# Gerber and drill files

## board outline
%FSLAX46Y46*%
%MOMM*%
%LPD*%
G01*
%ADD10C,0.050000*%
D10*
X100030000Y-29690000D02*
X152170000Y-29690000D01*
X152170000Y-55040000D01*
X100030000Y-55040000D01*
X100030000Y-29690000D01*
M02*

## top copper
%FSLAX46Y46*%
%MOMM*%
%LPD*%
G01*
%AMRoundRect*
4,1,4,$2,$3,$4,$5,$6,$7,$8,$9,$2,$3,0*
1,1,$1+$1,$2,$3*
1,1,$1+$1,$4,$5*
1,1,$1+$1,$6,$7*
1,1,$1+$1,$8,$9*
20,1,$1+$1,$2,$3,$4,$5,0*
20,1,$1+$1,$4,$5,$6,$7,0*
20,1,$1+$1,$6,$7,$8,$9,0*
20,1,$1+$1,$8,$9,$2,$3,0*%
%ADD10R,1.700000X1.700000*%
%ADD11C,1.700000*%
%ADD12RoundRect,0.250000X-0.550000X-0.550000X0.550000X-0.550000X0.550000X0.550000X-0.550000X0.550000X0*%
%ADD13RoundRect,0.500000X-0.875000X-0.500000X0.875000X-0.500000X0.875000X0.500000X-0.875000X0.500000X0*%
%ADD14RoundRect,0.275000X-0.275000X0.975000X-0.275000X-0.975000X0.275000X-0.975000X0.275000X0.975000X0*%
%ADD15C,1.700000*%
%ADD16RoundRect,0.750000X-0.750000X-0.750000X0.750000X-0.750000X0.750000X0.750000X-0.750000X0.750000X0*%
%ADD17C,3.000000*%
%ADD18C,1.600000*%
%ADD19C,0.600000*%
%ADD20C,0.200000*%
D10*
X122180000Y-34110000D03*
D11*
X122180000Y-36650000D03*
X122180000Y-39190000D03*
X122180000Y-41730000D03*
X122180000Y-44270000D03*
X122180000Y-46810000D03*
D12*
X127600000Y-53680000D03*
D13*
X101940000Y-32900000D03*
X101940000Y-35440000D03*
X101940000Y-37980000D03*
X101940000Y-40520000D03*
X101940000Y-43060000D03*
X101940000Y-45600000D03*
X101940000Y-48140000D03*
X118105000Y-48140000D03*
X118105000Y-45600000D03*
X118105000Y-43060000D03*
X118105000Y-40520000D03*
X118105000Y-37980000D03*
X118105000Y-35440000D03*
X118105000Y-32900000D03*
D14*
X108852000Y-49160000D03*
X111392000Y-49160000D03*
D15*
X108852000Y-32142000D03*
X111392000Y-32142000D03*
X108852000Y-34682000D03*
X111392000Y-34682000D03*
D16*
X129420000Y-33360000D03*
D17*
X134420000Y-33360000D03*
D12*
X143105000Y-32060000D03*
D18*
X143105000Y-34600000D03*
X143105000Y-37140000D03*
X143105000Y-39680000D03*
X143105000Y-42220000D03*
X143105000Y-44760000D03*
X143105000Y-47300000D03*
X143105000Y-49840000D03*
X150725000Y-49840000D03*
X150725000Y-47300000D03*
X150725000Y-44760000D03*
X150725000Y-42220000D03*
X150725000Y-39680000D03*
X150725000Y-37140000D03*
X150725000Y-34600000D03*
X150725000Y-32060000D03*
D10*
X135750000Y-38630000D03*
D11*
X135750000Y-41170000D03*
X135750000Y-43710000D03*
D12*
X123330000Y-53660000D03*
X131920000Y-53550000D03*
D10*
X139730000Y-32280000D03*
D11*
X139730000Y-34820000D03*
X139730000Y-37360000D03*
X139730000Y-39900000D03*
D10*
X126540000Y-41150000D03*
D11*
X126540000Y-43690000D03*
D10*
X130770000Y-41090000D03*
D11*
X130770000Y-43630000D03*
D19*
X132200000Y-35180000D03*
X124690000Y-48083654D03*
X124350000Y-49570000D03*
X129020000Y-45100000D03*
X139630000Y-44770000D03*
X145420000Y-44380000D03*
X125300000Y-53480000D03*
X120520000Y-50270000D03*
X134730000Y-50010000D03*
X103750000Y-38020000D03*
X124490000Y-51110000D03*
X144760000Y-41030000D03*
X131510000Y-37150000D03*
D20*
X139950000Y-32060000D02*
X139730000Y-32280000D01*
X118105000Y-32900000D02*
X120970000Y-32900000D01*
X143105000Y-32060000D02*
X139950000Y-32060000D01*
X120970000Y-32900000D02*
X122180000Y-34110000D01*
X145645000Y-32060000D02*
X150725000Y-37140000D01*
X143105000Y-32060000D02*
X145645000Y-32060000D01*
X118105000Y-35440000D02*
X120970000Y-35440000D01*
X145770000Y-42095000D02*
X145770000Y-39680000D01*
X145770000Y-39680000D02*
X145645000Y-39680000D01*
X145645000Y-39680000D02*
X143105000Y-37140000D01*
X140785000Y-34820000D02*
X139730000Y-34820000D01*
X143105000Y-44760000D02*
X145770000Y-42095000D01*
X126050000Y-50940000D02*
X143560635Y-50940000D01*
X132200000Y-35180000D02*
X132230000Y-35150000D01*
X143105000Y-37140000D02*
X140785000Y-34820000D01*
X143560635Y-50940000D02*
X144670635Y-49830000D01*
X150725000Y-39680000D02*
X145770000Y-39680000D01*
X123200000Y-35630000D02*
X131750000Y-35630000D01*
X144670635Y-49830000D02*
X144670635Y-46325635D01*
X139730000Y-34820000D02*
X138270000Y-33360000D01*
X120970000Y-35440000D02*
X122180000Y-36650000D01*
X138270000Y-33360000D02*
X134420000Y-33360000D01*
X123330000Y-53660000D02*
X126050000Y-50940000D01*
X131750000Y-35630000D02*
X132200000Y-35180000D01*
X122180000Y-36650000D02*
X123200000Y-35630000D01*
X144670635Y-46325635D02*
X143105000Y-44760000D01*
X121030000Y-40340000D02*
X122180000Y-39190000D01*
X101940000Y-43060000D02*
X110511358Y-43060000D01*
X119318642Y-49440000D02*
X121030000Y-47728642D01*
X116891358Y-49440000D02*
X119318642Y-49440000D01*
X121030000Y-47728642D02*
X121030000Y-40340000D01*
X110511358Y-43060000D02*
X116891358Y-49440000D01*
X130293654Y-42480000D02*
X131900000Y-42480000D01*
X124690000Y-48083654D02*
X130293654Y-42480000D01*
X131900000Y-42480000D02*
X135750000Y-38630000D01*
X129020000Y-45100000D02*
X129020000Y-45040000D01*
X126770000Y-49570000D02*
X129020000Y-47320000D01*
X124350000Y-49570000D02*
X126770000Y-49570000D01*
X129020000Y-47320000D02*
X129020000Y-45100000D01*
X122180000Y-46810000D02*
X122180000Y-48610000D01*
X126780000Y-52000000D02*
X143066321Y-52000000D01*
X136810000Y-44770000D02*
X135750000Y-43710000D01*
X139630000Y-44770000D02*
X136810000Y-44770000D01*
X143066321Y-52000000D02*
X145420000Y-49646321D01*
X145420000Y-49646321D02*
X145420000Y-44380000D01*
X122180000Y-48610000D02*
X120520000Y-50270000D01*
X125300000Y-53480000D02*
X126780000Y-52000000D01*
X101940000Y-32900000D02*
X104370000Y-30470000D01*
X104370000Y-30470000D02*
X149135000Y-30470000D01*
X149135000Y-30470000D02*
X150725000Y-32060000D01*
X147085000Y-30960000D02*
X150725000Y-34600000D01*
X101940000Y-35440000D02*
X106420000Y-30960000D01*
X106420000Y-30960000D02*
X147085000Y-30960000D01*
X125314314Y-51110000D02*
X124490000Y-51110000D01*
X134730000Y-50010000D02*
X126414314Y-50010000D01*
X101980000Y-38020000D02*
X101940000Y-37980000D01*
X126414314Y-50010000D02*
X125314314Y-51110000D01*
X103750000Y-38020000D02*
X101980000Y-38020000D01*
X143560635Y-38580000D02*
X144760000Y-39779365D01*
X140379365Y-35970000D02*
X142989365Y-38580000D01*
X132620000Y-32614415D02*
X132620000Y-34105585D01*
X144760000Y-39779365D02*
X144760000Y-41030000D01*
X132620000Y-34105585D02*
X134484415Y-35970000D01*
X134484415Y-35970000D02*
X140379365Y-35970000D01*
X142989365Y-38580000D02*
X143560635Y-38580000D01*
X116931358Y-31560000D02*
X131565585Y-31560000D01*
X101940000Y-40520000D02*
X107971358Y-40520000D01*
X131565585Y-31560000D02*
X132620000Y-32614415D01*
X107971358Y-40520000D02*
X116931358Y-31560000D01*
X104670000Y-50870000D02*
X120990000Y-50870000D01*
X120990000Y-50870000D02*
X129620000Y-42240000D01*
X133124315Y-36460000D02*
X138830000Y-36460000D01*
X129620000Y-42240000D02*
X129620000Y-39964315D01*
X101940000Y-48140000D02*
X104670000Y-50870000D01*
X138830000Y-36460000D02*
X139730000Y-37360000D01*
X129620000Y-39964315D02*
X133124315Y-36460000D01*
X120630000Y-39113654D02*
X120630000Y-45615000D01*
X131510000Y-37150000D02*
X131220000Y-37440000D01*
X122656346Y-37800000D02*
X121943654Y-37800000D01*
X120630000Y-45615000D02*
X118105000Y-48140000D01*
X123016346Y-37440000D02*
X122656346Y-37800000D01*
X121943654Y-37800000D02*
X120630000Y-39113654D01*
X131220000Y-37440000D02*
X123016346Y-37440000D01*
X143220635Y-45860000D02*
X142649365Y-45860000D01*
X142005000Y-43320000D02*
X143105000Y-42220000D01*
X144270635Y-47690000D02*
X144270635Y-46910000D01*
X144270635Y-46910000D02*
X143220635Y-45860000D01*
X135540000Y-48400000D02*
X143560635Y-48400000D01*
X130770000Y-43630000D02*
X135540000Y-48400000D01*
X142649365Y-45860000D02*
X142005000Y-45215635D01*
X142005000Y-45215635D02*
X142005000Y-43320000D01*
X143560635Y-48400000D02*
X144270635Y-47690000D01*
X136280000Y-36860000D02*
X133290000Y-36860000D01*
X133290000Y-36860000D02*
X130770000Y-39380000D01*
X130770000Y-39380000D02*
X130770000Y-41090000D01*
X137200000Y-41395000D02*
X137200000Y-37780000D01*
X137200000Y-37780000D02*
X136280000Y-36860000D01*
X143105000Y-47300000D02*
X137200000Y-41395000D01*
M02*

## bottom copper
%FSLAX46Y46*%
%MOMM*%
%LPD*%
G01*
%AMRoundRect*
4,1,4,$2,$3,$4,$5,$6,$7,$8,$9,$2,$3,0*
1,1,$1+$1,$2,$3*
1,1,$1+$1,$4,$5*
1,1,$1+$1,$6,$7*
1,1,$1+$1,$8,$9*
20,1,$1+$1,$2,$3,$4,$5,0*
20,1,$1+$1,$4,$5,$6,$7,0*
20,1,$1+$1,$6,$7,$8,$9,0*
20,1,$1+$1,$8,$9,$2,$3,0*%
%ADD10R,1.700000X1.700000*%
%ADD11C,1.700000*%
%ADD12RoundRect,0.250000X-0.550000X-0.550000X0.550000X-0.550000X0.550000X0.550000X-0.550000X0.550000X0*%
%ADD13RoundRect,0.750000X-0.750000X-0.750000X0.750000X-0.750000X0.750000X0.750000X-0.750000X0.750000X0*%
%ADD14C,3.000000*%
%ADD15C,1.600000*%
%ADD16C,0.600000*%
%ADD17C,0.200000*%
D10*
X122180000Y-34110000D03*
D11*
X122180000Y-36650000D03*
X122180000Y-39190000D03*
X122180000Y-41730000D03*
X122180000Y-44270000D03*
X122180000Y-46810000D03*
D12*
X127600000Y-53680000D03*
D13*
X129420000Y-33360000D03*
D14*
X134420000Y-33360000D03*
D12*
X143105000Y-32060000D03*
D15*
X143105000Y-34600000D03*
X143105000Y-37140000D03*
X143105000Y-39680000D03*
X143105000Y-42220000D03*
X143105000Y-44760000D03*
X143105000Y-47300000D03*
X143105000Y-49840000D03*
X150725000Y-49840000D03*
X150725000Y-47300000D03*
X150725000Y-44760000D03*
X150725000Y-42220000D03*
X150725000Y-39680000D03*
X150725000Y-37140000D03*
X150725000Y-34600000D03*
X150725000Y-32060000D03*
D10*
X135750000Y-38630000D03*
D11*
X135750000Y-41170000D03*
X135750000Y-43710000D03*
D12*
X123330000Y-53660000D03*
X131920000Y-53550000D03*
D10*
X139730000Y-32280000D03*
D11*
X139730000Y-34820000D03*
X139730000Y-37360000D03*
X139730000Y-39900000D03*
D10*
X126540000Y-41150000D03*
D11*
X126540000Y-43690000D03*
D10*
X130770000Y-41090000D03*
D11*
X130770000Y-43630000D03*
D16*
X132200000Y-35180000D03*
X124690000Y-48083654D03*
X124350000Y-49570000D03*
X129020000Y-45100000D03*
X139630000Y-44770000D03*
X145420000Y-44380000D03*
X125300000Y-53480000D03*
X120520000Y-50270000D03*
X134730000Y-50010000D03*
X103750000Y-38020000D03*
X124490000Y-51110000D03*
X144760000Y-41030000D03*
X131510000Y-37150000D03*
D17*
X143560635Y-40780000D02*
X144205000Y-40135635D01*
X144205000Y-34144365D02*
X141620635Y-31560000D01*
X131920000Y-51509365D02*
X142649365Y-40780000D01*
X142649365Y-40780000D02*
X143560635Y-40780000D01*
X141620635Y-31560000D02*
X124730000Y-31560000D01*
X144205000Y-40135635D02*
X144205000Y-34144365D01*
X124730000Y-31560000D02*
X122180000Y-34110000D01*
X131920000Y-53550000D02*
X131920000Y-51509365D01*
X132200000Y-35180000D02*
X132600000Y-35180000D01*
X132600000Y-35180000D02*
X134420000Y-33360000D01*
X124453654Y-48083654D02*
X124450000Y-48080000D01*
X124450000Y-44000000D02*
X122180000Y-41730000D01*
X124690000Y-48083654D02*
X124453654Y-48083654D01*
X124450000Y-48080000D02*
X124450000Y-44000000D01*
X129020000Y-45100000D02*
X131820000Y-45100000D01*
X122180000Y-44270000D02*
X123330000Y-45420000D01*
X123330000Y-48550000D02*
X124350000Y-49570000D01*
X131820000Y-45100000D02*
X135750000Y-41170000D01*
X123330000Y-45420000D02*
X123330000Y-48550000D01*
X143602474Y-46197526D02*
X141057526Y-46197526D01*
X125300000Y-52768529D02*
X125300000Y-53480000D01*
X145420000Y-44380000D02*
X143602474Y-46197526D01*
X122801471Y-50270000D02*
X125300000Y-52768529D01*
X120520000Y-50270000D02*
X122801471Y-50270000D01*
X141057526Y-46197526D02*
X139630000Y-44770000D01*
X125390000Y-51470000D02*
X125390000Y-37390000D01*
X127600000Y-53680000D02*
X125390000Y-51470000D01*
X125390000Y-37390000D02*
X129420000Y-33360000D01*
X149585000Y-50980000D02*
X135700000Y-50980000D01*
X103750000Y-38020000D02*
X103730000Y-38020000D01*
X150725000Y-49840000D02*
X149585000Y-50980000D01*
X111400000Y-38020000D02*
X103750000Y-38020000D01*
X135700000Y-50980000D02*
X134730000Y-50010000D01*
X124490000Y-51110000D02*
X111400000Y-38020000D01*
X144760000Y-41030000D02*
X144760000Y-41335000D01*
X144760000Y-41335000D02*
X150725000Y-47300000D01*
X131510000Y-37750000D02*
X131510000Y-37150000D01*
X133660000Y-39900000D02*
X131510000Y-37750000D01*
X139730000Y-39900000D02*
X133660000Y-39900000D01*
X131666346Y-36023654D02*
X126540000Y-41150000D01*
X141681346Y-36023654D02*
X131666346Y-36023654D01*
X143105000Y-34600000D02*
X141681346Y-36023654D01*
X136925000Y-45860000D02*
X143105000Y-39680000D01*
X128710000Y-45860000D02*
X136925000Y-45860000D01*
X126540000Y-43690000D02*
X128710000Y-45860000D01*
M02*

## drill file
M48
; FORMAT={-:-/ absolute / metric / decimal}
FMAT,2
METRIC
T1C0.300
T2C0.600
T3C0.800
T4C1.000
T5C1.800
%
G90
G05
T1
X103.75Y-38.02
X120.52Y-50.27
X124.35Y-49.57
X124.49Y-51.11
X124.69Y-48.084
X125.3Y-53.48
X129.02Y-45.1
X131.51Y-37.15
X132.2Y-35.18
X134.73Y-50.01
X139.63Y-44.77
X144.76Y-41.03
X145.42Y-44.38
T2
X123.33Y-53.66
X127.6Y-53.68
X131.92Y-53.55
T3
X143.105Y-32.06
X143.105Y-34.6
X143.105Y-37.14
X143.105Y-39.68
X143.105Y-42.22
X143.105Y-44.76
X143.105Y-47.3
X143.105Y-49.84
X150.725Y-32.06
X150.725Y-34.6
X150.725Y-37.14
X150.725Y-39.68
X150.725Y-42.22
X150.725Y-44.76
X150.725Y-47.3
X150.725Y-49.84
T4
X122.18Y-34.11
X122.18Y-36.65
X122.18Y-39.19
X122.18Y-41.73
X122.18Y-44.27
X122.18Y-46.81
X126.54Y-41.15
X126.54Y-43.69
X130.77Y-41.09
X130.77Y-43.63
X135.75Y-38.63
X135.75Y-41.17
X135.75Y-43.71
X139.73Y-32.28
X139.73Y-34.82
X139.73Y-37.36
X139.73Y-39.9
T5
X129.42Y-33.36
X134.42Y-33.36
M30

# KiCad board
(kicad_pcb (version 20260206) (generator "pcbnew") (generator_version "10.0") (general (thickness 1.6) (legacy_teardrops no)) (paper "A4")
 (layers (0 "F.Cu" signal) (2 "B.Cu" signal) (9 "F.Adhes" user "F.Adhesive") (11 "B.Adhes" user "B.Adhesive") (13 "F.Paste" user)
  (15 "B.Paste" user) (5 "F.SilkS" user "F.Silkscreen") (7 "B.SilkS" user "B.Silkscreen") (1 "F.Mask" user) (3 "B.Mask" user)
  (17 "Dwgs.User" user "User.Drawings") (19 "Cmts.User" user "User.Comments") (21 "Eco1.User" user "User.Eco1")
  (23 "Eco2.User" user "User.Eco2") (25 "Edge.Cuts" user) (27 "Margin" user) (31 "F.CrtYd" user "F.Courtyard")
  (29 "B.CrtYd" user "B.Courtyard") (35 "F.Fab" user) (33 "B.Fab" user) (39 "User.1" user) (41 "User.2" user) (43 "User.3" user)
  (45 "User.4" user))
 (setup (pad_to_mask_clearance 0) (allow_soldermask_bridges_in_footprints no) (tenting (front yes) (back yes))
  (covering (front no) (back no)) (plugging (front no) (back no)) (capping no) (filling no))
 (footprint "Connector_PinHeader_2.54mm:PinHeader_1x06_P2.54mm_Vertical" (layer "F.Cu") (at 122.18 34.11)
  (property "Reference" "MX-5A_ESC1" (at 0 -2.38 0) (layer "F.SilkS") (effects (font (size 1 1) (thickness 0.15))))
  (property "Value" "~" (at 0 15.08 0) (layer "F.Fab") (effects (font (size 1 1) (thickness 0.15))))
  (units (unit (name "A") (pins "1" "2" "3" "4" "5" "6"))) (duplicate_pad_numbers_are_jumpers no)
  (pad "1" thru_hole rect (at 0 0) (size 1.7 1.7) (drill 1) (layers "*.Cu" "*.Mask") (remove_unused_layers no) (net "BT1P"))
  (pad "2" thru_hole circle (at 0 2.54) (size 1.7 1.7) (drill 1) (layers "*.Cu" "*.Mask") (remove_unused_layers no) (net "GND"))
  (pad "3" thru_hole circle (at 0 5.08) (size 1.7 1.7) (drill 1) (layers "*.Cu" "*.Mask") (remove_unused_layers no)
   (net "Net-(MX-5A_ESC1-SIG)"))
  (pad "4" thru_hole circle (at 0 7.62) (size 1.7 1.7) (drill 1) (layers "*.Cu" "*.Mask") (remove_unused_layers no)
   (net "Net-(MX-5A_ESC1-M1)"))
  (pad "5" thru_hole circle (at 0 10.16) (size 1.7 1.7) (drill 1) (layers "*.Cu" "*.Mask") (remove_unused_layers no)
   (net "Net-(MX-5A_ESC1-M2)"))
  (pad "6" thru_hole circle (at 0 12.7) (size 1.7 1.7) (drill 1) (layers "*.Cu" "*.Mask") (remove_unused_layers no)
   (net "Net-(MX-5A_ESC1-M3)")))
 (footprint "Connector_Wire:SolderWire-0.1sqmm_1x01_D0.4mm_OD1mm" (layer "F.Cu") (at 127.6 53.68)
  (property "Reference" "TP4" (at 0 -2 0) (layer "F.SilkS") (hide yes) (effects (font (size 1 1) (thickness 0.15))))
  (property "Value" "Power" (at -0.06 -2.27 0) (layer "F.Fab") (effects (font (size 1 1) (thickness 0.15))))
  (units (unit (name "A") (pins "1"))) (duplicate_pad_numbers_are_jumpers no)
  (pad "1" thru_hole roundrect (at 0 0) (size 1.6 1.6) (drill 0.6) (layers "*.Cu" "*.Mask") (remove_unused_layers no)
   (roundrect_rratio 0.15625) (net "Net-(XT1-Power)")))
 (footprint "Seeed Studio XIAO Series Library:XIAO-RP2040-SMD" (layer "F.Cu") (at 109.94 40.52)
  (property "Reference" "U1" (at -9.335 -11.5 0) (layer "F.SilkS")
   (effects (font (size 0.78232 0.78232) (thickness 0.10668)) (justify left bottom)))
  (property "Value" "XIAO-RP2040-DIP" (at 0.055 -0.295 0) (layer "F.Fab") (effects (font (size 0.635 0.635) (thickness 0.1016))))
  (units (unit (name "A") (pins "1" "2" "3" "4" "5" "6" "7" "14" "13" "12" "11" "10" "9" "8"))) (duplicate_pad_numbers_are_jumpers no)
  (pad "1" smd roundrect (at -8 -7.62) (size 2.75 2) (layers "F.Cu" "F.Mask" "F.Paste") (roundrect_rratio 0.25) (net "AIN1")
   (solder_mask_margin 0.0508) (thermal_bridge_angle 45))
  (pad "2" smd roundrect (at -8 -5.08) (size 2.75 2) (layers "F.Cu" "F.Mask" "F.Paste") (roundrect_rratio 0.25) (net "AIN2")
   (solder_mask_margin 0.0508) (thermal_bridge_angle 45))
  (pad "3" smd roundrect (at -8 -2.54) (size 2.75 2) (layers "F.Cu" "F.Mask" "F.Paste") (roundrect_rratio 0.25) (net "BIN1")
   (solder_mask_margin 0.0508) (thermal_bridge_angle 45))
  (pad "4" smd roundrect (at -8 0) (size 2.75 2) (layers "F.Cu" "F.Mask" "F.Paste") (roundrect_rratio 0.25) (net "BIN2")
   (solder_mask_margin 0.0508) (thermal_bridge_angle 45))
  (pad "5" smd roundrect (at -8 2.54) (size 2.75 2) (layers "F.Cu" "F.Mask" "F.Paste") (roundrect_rratio 0.25) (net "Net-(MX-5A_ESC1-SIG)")
   (solder_mask_margin 0.0508) (thermal_bridge_angle 45))
  (pad "6" smd roundrect (at -8 5.08) (size 2.75 2) (layers "F.Cu" "F.Mask" "F.Paste") (roundrect_rratio 0.25)
   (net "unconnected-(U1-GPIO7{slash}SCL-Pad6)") (solder_mask_margin 0.0508) (thermal_bridge_angle 45))
  (pad "7" smd roundrect (at -8 7.62) (size 2.75 2) (layers "F.Cu" "F.Mask" "F.Paste") (roundrect_rratio 0.25)
   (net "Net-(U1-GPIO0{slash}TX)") (solder_mask_margin 0.0508) (thermal_bridge_angle 45))
  (pad "8" smd roundrect (at 8.165 7.62) (size 2.75 2) (layers "F.Cu" "F.Mask" "F.Paste") (roundrect_rratio 0.25)
   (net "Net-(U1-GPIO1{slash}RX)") (solder_mask_margin 0.0508) (thermal_bridge_angle 45))
  (pad "9" smd roundrect (at 8.165 5.08) (size 2.75 2) (layers "F.Cu" "F.Mask" "F.Paste") (roundrect_rratio 0.25)
   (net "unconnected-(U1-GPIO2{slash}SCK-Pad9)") (solder_mask_margin 0.0508) (thermal_bridge_angle 45))
  (pad "10" smd roundrect (at 8.165 2.54) (size 2.75 2) (layers "F.Cu" "F.Mask" "F.Paste") (roundrect_rratio 0.25)
   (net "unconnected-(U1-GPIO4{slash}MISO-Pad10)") (solder_mask_margin 0.0508) (thermal_bridge_angle 45))
  (pad "11" smd roundrect (at 8.165 0) (size 2.75 2) (layers "F.Cu" "F.Mask" "F.Paste") (roundrect_rratio 0.25)
   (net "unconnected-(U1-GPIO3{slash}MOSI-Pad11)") (solder_mask_margin 0.0508) (thermal_bridge_angle 45))
  (pad "12" smd roundrect (at 8.165 -2.54) (size 2.75 2) (layers "F.Cu" "F.Mask" "F.Paste") (roundrect_rratio 0.25)
   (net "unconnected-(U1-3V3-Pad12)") (solder_mask_margin 0.0508) (thermal_bridge_angle 45))
  (pad "13" smd roundrect (at 8.165 -5.08) (size 2.75 2) (layers "F.Cu" "F.Mask" "F.Paste") (roundrect_rratio 0.25) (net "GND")
   (solder_mask_margin 0.0508) (thermal_bridge_angle 45))
  (pad "14" smd roundrect (at 8.165 -7.62) (size 2.75 2) (layers "F.Cu" "F.Mask" "F.Paste") (roundrect_rratio 0.25) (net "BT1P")
   (solder_mask_margin 0.0508) (thermal_bridge_angle 45))
  (pad "15" smd roundrect (at -1.088 8.64 270) (size 2.5 1.1) (layers "F.Cu" "F.Mask" "F.Paste") (roundrect_rratio 0.25)
   (thermal_bridge_angle 45))
  (pad "16" smd roundrect (at 1.452 8.64 270) (size 2.5 1.1) (layers "F.Cu" "F.Mask" "F.Paste") (roundrect_rratio 0.25)
   (thermal_bridge_angle 45))
  (pad "17" smd circle (at -1.088 -8.378) (size 1.7 1.7) (layers "F.Cu" "F.Mask" "F.Paste"))
  (pad "18" smd circle (at 1.452 -8.378) (size 1.7 1.7) (layers "F.Cu" "F.Mask" "F.Paste"))
  (pad "19" smd circle (at -1.088 -5.838) (size 1.7 1.7) (layers "F.Cu" "F.Mask" "F.Paste"))
  (pad "20" smd circle (at 1.452 -5.838) (size 1.7 1.7) (layers "F.Cu" "F.Mask" "F.Paste")))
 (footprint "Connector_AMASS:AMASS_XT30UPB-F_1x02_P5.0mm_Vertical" (layer "F.Cu") (at 129.42 33.36)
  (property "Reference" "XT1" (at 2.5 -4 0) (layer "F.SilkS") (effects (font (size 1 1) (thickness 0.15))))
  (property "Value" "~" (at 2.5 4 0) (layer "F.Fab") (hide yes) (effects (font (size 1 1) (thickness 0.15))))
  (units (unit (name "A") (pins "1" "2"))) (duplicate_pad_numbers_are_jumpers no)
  (pad "1" thru_hole roundrect (at 0 0) (size 3 3) (drill 1.8) (layers "*.Cu" "*.Mask") (remove_unused_layers no) (roundrect_rratio 0.25)
   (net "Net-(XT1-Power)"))
  (pad "2" thru_hole circle (at 5 0) (size 3 3) (drill 1.8) (layers "*.Cu" "*.Mask") (remove_unused_layers no) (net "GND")))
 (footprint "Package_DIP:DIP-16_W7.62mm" (layer "F.Cu") (at 143.105 32.06)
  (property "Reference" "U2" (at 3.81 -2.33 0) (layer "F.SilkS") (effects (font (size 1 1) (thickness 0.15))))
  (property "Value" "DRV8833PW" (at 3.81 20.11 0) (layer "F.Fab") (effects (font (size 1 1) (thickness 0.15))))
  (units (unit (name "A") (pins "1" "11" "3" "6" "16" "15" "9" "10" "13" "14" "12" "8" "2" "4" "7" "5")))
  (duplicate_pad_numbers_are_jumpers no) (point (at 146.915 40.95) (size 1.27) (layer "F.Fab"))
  (pad "1" thru_hole roundrect (at 0 0) (size 1.6 1.6) (drill 0.8) (layers "*.Cu" "*.Mask") (remove_unused_layers no)
   (roundrect_rratio 0.15625) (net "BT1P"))
  (pad "2" thru_hole circle (at 0 2.54) (size 1.6 1.6) (drill 0.8) (layers "*.Cu" "*.Mask") (remove_unused_layers no) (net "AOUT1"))
  (pad "3" thru_hole circle (at 0 5.08) (size 1.6 1.6) (drill 0.8) (layers "*.Cu" "*.Mask") (remove_unused_layers no) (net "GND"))
  (pad "4" thru_hole circle (at 0 7.62) (size 1.6 1.6) (drill 0.8) (layers "*.Cu" "*.Mask") (remove_unused_layers no) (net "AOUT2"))
  (pad "5" thru_hole circle (at 0 10.16) (size 1.6 1.6) (drill 0.8) (layers "*.Cu" "*.Mask") (remove_unused_layers no) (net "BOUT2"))
  (pad "6" thru_hole circle (at 0 12.7) (size 1.6 1.6) (drill 0.8) (layers "*.Cu" "*.Mask") (remove_unused_layers no) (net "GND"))
  (pad "7" thru_hole circle (at 0 15.24) (size 1.6 1.6) (drill 0.8) (layers "*.Cu" "*.Mask") (remove_unused_layers no) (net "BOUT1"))
  (pad "8" thru_hole circle (at 0 17.78) (size 1.6 1.6) (drill 0.8) (layers "*.Cu" "*.Mask") (remove_unused_layers no)
   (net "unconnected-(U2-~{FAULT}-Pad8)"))
  (pad "9" thru_hole circle (at 7.62 17.78) (size 1.6 1.6) (drill 0.8) (layers "*.Cu" "*.Mask") (remove_unused_layers no) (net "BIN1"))
  (pad "10" thru_hole circle (at 7.62 15.24) (size 1.6 1.6) (drill 0.8) (layers "*.Cu" "*.Mask") (remove_unused_layers no) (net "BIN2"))
  (pad "11" thru_hole circle (at 7.62 12.7) (size 1.6 1.6) (drill 0.8) (layers "*.Cu" "*.Mask") (remove_unused_layers no)
   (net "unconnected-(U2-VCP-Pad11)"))
  (pad "12" thru_hole circle (at 7.62 10.16) (size 1.6 1.6) (drill 0.8) (layers "*.Cu" "*.Mask") (remove_unused_layers no)
   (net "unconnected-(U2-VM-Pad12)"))
  (pad "13" thru_hole circle (at 7.62 7.62) (size 1.6 1.6) (drill 0.8) (layers "*.Cu" "*.Mask") (remove_unused_layers no) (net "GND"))
  (pad "14" thru_hole circle (at 7.62 5.08) (size 1.6 1.6) (drill 0.8) (layers "*.Cu" "*.Mask") (remove_unused_layers no) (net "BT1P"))
  (pad "15" thru_hole circle (at 7.62 2.54) (size 1.6 1.6) (drill 0.8) (layers "*.Cu" "*.Mask") (remove_unused_layers no) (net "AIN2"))
  (pad "16" thru_hole circle (at 7.62 0) (size 1.6 1.6) (drill 0.8) (layers "*.Cu" "*.Mask") (remove_unused_layers no) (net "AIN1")))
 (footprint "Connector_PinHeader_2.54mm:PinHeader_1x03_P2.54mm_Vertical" (layer "F.Cu") (at 135.75 38.63)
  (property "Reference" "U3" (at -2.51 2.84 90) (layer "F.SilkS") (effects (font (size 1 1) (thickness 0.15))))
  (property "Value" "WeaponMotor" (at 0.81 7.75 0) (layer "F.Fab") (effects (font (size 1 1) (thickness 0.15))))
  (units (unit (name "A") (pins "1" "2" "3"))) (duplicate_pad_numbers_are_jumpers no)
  (pad "1" thru_hole rect (at 0 0) (size 1.7 1.7) (drill 1) (layers "*.Cu" "*.Mask") (remove_unused_layers no) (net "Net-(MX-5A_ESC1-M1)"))
  (pad "2" thru_hole circle (at 0 2.54) (size 1.7 1.7) (drill 1) (layers "*.Cu" "*.Mask") (remove_unused_layers no)
   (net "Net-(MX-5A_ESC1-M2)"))
  (pad "3" thru_hole circle (at 0 5.08) (size 1.7 1.7) (drill 1) (layers "*.Cu" "*.Mask") (remove_unused_layers no)
   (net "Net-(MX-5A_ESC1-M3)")))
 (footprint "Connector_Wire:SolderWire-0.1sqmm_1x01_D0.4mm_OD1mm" (layer "F.Cu") (at 123.33 53.66)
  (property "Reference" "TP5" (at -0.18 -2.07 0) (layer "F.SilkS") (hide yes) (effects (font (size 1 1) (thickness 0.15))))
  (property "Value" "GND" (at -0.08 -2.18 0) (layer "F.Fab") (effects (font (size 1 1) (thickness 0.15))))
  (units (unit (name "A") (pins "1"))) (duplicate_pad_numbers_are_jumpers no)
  (pad "1" thru_hole roundrect (at 0 0) (size 1.6 1.6) (drill 0.6) (layers "*.Cu" "*.Mask") (remove_unused_layers no)
   (roundrect_rratio 0.15625) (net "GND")))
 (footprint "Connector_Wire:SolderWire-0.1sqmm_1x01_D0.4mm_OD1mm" (layer "F.Cu") (at 131.92 53.55)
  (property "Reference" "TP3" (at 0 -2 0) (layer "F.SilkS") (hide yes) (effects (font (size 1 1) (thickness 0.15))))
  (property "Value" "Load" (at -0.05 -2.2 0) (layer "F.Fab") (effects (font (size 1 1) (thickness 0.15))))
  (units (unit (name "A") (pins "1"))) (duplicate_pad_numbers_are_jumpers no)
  (pad "1" thru_hole roundrect (at 0 0) (size 1.6 1.6) (drill 0.6) (layers "*.Cu" "*.Mask") (remove_unused_layers no)
   (roundrect_rratio 0.15625) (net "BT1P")))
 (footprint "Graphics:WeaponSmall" (layer "F.Cu") (at 103.49791 55.032445 90)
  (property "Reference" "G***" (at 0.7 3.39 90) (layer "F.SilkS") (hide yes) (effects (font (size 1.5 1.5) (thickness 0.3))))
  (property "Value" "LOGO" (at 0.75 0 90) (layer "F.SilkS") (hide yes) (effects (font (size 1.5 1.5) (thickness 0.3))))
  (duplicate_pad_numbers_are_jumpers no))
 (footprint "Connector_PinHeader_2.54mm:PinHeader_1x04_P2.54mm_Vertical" (layer "F.Cu") (at 139.73 32.28)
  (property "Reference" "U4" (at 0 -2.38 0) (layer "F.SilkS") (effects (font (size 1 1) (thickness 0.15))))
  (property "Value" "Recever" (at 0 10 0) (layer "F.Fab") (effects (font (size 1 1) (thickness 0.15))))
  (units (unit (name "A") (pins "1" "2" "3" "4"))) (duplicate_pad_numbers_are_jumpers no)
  (pad "1" thru_hole rect (at 0 0) (size 1.7 1.7) (drill 1) (layers "*.Cu" "*.Mask") (remove_unused_layers no) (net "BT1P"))
  (pad "2" thru_hole circle (at 0 2.54) (size 1.7 1.7) (drill 1) (layers "*.Cu" "*.Mask") (remove_unused_layers no) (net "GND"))
  (pad "3" thru_hole circle (at 0 5.08) (size 1.7 1.7) (drill 1) (layers "*.Cu" "*.Mask") (remove_unused_layers no)
   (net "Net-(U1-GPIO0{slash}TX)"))
  (pad "4" thru_hole circle (at 0 7.62) (size 1.7 1.7) (drill 1) (layers "*.Cu" "*.Mask") (remove_unused_layers no)
   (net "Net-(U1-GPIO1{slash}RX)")))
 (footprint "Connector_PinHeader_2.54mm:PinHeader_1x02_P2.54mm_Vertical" (layer "F.Cu") (at 126.54 41.15)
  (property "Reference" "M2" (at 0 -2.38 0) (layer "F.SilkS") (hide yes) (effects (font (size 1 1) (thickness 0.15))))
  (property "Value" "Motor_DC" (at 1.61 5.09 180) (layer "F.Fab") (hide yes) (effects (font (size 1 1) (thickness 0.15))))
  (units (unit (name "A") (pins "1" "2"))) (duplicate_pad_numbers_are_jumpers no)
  (pad "1" thru_hole rect (at 0 0) (size 1.7 1.7) (drill 1) (layers "*.Cu" "*.Mask") (remove_unused_layers no) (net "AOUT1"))
  (pad "2" thru_hole circle (at 0 2.54) (size 1.7 1.7) (drill 1) (layers "*.Cu" "*.Mask") (remove_unused_layers no) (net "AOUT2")))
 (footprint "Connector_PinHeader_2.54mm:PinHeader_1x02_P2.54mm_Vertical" (layer "F.Cu") (at 130.77 41.09)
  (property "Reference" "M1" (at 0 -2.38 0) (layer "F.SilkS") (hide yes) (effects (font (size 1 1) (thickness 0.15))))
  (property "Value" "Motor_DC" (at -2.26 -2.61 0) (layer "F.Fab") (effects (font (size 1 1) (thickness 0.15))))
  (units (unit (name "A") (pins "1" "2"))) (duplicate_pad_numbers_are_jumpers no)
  (pad "1" thru_hole rect (at 0 0) (size 1.7 1.7) (drill 1) (layers "*.Cu" "*.Mask") (remove_unused_layers no) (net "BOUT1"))
  (pad "2" thru_hole circle (at 0 2.54) (size 1.7 1.7) (drill 1) (layers "*.Cu" "*.Mask") (remove_unused_layers no) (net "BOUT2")))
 (gr_rect (start 100.03 29.69) (end 152.17 55.04) (stroke (width 0.05) (type default)) (fill no) (layer "Edge.Cuts"))
 (segment (start 139.95 32.06) (end 139.73 32.28) (width 0.2) (layer "F.Cu") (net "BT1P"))
 (segment (start 118.105 32.9) (end 120.97 32.9) (width 0.2) (layer "F.Cu") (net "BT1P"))
 (segment (start 143.105 32.06) (end 139.95 32.06) (width 0.2) (layer "F.Cu") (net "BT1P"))
 (segment (start 120.97 32.9) (end 122.18 34.11) (width 0.2) (layer "F.Cu") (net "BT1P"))
 (segment (start 145.645 32.06) (end 150.725 37.14) (width 0.2) (layer "F.Cu") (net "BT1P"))
 (segment (start 143.105 32.06) (end 145.645 32.06) (width 0.2) (layer "F.Cu") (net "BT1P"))
 (segment (start 143.560635 40.78) (end 144.205 40.135635) (width 0.2) (layer "B.Cu") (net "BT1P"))
 (segment (start 144.205 34.144365) (end 141.620635 31.56) (width 0.2) (layer "B.Cu") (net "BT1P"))
 (segment (start 131.92 51.509365) (end 142.649365 40.78) (width 0.2) (layer "B.Cu") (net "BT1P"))
 (segment (start 142.649365 40.78) (end 143.560635 40.78) (width 0.2) (layer "B.Cu") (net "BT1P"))
 (segment (start 141.620635 31.56) (end 124.73 31.56) (width 0.2) (layer "B.Cu") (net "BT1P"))
 (segment (start 144.205 40.135635) (end 144.205 34.144365) (width 0.2) (layer "B.Cu") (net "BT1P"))
 (segment (start 124.73 31.56) (end 122.18 34.11) (width 0.2) (layer "B.Cu") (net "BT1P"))
 (segment (start 131.92 53.55) (end 131.92 51.509365) (width 0.2) (layer "B.Cu") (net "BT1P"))
 (segment (start 118.105 35.44) (end 120.97 35.44) (width 0.2) (layer "F.Cu") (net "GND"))
 (segment (start 145.77 42.095) (end 145.77 39.68) (width 0.2) (layer "F.Cu") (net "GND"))
 (segment (start 145.77 39.68) (end 145.645 39.68) (width 0.2) (layer "F.Cu") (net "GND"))
 (segment (start 145.645 39.68) (end 143.105 37.14) (width 0.2) (layer "F.Cu") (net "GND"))
 (segment (start 140.785 34.82) (end 139.73 34.82) (width 0.2) (layer "F.Cu") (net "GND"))
 (segment (start 143.105 44.76) (end 145.77 42.095) (width 0.2) (layer "F.Cu") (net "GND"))
 (segment (start 126.05 50.94) (end 143.560635 50.94) (width 0.2) (layer "F.Cu") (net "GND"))
 (segment (start 132.2 35.18) (end 132.23 35.15) (width 0.2) (layer "F.Cu") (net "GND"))
 (segment (start 143.105 37.14) (end 140.785 34.82) (width 0.2) (layer "F.Cu") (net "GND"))
 (segment (start 143.560635 50.94) (end 144.670635 49.83) (width 0.2) (layer "F.Cu") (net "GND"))
 (segment (start 150.725 39.68) (end 145.77 39.68) (width 0.2) (layer "F.Cu") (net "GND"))
 (segment (start 123.2 35.63) (end 131.75 35.63) (width 0.2) (layer "F.Cu") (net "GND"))
 (segment (start 144.670635 49.83) (end 144.670635 46.325635) (width 0.2) (layer "F.Cu") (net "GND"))
 (segment (start 139.73 34.82) (end 138.27 33.36) (width 0.2) (layer "F.Cu") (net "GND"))
 (segment (start 120.97 35.44) (end 122.18 36.65) (width 0.2) (layer "F.Cu") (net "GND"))
 (segment (start 138.27 33.36) (end 134.42 33.36) (width 0.2) (layer "F.Cu") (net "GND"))
 (segment (start 123.33 53.66) (end 126.05 50.94) (width 0.2) (layer "F.Cu") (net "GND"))
 (segment (start 131.75 35.63) (end 132.2 35.18) (width 0.2) (layer "F.Cu") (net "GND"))
 (segment (start 122.18 36.65) (end 123.2 35.63) (width 0.2) (layer "F.Cu") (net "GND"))
 (segment (start 144.670635 46.325635) (end 143.105 44.76) (width 0.2) (layer "F.Cu") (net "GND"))
 (via (at 132.2 35.18) (size 0.6) (drill 0.3) (layers "F.Cu" "B.Cu") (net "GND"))
 (segment (start 132.2 35.18) (end 132.6 35.18) (width 0.2) (layer "B.Cu") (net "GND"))
 (segment (start 132.6 35.18) (end 134.42 33.36) (width 0.2) (layer "B.Cu") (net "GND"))
 (segment (start 121.03 40.34) (end 122.18 39.19) (width 0.2) (layer "F.Cu") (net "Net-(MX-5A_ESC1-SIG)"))
 (segment (start 101.94 43.06) (end 110.511358 43.06) (width 0.2) (layer "F.Cu") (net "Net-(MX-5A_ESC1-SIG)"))
 (segment (start 119.318642 49.44) (end 121.03 47.728642) (width 0.2) (layer "F.Cu") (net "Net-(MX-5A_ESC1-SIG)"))
 (segment (start 116.891358 49.44) (end 119.318642 49.44) (width 0.2) (layer "F.Cu") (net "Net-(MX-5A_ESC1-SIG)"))
 (segment (start 121.03 47.728642) (end 121.03 40.34) (width 0.2) (layer "F.Cu") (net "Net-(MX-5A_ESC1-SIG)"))
 (segment (start 110.511358 43.06) (end 116.891358 49.44) (width 0.2) (layer "F.Cu") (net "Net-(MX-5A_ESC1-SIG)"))
 (segment (start 130.293654 42.48) (end 131.9 42.48) (width 0.2) (layer "F.Cu") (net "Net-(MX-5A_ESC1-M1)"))
 (segment (start 124.69 48.083654) (end 130.293654 42.48) (width 0.2) (layer "F.Cu") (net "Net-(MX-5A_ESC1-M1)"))
 (segment (start 131.9 42.48) (end 135.75 38.63) (width 0.2) (layer "F.Cu") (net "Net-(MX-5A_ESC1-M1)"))
 (via (at 124.69 48.083654) (size 0.6) (drill 0.3) (layers "F.Cu" "B.Cu") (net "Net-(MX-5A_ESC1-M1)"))
 (segment (start 124.453654 48.083654) (end 124.45 48.08) (width 0.2) (layer "B.Cu") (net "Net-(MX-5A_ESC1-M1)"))
 (segment (start 124.45 44) (end 122.18 41.73) (width 0.2) (layer "B.Cu") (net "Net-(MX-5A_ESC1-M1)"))
 (segment (start 124.69 48.083654) (end 124.453654 48.083654) (width 0.2) (layer "B.Cu") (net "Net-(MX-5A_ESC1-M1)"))
 (segment (start 124.45 48.08) (end 124.45 44) (width 0.2) (layer "B.Cu") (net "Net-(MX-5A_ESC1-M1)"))
 (segment (start 129.02 45.1) (end 129.02 45.04) (width 0.2) (layer "F.Cu") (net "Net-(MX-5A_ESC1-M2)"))
 (segment (start 126.77 49.57) (end 129.02 47.32) (width 0.2) (layer "F.Cu") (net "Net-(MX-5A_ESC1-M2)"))
 (segment (start 124.35 49.57) (end 126.77 49.57) (width 0.2) (layer "F.Cu") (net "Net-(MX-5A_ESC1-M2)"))
 (segment (start 129.02 47.32) (end 129.02 45.1) (width 0.2) (layer "F.Cu") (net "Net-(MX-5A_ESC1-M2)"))
 (via (at 124.35 49.57) (size 0.6) (drill 0.3) (layers "F.Cu" "B.Cu") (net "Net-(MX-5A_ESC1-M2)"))
 (via (at 129.02 45.1) (size 0.6) (drill 0.3) (layers "F.Cu" "B.Cu") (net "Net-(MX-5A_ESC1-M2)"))
 (segment (start 129.02 45.1) (end 131.82 45.1) (width 0.2) (layer "B.Cu") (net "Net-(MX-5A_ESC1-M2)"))
 (segment (start 122.18 44.27) (end 123.33 45.42) (width 0.2) (layer "B.Cu") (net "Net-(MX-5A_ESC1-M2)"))
 (segment (start 123.33 48.55) (end 124.35 49.57) (width 0.2) (layer "B.Cu") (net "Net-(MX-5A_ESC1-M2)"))
 (segment (start 131.82 45.1) (end 135.75 41.17) (width 0.2) (layer "B.Cu") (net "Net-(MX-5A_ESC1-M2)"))
 (segment (start 123.33 45.42) (end 123.33 48.55) (width 0.2) (layer "B.Cu") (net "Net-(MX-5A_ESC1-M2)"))
 (segment (start 122.18 46.81) (end 122.18 48.61) (width 0.2) (layer "F.Cu") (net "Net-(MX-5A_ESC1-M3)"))
 (segment (start 126.78 52) (end 143.066321 52) (width 0.2) (layer "F.Cu") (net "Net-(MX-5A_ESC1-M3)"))
 (segment (start 136.81 44.77) (end 135.75 43.71) (width 0.2) (layer "F.Cu") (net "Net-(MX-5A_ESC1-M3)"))
 (segment (start 139.63 44.77) (end 136.81 44.77) (width 0.2) (layer "F.Cu") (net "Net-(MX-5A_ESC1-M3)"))
 (segment (start 143.066321 52) (end 145.42 49.646321) (width 0.2) (layer "F.Cu") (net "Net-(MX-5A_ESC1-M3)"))
 (segment (start 145.42 49.646321) (end 145.42 44.38) (width 0.2) (layer "F.Cu") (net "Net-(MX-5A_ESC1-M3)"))
 (segment (start 122.18 48.61) (end 120.52 50.27) (width 0.2) (layer "F.Cu") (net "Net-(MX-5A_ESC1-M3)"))
 (segment (start 125.3 53.48) (end 126.78 52) (width 0.2) (layer "F.Cu") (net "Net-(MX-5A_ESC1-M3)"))
 (via (at 139.63 44.77) (size 0.6) (drill 0.3) (layers "F.Cu" "B.Cu") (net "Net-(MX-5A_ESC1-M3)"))
 (via (at 145.42 44.38) (size 0.6) (drill 0.3) (layers "F.Cu" "B.Cu") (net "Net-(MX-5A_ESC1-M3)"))
 (via (at 125.3 53.48) (size 0.6) (drill 0.3) (layers "F.Cu" "B.Cu") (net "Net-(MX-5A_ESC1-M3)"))
 (via (at 120.52 50.27) (size 0.6) (drill 0.3) (layers "F.Cu" "B.Cu") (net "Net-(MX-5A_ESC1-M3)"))
 (segment (start 143.602474 46.197526) (end 141.057526 46.197526) (width 0.2) (layer "B.Cu") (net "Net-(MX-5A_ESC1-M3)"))
 (segment (start 125.3 52.768529) (end 125.3 53.48) (width 0.2) (layer "B.Cu") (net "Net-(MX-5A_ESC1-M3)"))
 (segment (start 145.42 44.38) (end 143.602474 46.197526) (width 0.2) (layer "B.Cu") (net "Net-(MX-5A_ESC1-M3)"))
 (segment (start 122.801471 50.27) (end 125.3 52.768529) (width 0.2) (layer "B.Cu") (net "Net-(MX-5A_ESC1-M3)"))
 (segment (start 120.52 50.27) (end 122.801471 50.27) (width 0.2) (layer "B.Cu") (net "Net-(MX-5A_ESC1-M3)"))
 (segment (start 141.057526 46.197526) (end 139.63 44.77) (width 0.2) (layer "B.Cu") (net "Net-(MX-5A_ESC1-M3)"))
 (segment (start 125.39 51.47) (end 125.39 37.39) (width 0.2) (layer "B.Cu") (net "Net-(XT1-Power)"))
 (segment (start 127.6 53.68) (end 125.39 51.47) (width 0.2) (layer "B.Cu") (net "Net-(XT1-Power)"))
 (segment (start 125.39 37.39) (end 129.42 33.36) (width 0.2) (layer "B.Cu") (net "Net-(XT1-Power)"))
 (segment (start 101.94 32.9) (end 104.37 30.47) (width 0.2) (layer "F.Cu") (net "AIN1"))
 (segment (start 104.37 30.47) (end 149.135 30.47) (width 0.2) (layer "F.Cu") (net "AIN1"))
 (segment (start 149.135 30.47) (end 150.725 32.06) (width 0.2) (layer "F.Cu") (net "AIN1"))
 (segment (start 147.085 30.96) (end 150.725 34.6) (width 0.2) (layer "F.Cu") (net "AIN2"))
 (segment (start 101.94 35.44) (end 106.42 30.96) (width 0.2) (layer "F.Cu") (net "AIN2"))
 (segment (start 106.42 30.96) (end 147.085 30.96) (width 0.2) (layer "F.Cu") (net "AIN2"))
 (segment (start 125.314314 51.11) (end 124.49 51.11) (width 0.2) (layer "F.Cu") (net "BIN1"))
 (segment (start 134.73 50.01) (end 126.414314 50.01) (width 0.2) (layer "F.Cu") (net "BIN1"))
 (segment (start 101.98 38.02) (end 101.94 37.98) (width 0.2) (layer "F.Cu") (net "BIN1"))
 (segment (start 126.414314 50.01) (end 125.314314 51.11) (width 0.2) (layer "F.Cu") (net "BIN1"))
 (segment (start 103.75 38.02) (end 101.98 38.02) (width 0.2) (layer "F.Cu") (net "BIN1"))
 (via (at 134.73 50.01) (size 0.6) (drill 0.3) (layers "F.Cu" "B.Cu") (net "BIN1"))
 (via (at 103.75 38.02) (size 0.6) (drill 0.3) (layers "F.Cu" "B.Cu") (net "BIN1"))
 (via (at 124.49 51.11) (size 0.6) (drill 0.3) (layers "F.Cu" "B.Cu") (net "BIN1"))
 (segment (start 149.585 50.98) (end 135.7 50.98) (width 0.2) (layer "B.Cu") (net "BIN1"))
 (segment (start 103.75 38.02) (end 103.73 38.02) (width 0.2) (layer "B.Cu") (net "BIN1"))
 (segment (start 150.725 49.84) (end 149.585 50.98) (width 0.2) (layer "B.Cu") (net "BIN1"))
 (segment (start 111.4 38.02) (end 103.75 38.02) (width 0.2) (layer "B.Cu") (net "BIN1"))
 (segment (start 135.7 50.98) (end 134.73 50.01) (width 0.2) (layer "B.Cu") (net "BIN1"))
 (segment (start 124.49 51.11) (end 111.4 38.02) (width 0.2) (layer "B.Cu") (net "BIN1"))
 (segment (start 143.560635 38.58) (end 144.76 39.779365) (width 0.2) (layer "F.Cu") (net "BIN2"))
 (segment (start 140.379365 35.97) (end 142.989365 38.58) (width 0.2) (layer "F.Cu") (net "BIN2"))
 (segment (start 132.62 32.614415) (end 132.62 34.105585) (width 0.2) (layer "F.Cu") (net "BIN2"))
 (segment (start 144.76 39.779365) (end 144.76 41.03) (width 0.2) (layer "F.Cu") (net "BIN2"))
 (segment (start 132.62 34.105585) (end 134.484415 35.97) (width 0.2) (layer "F.Cu") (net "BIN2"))
 (segment (start 134.484415 35.97) (end 140.379365 35.97) (width 0.2) (layer "F.Cu") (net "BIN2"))
 (segment (start 142.989365 38.58) (end 143.560635 38.58) (width 0.2) (layer "F.Cu") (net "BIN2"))
 (segment (start 116.931358 31.56) (end 131.565585 31.56) (width 0.2) (layer "F.Cu") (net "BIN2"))
 (segment (start 101.94 40.52) (end 107.971358 40.52) (width 0.2) (layer "F.Cu") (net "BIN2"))
 (segment (start 131.565585 31.56) (end 132.62 32.614415) (width 0.2) (layer "F.Cu") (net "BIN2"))
 (segment (start 107.971358 40.52) (end 116.931358 31.56) (width 0.2) (layer "F.Cu") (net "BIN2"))
 (via (at 144.76 41.03) (size 0.6) (drill 0.3) (layers "F.Cu" "B.Cu") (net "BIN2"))
 (segment (start 144.76 41.03) (end 144.76 41.335) (width 0.2) (layer "B.Cu") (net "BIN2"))
 (segment (start 144.76 41.335) (end 150.725 47.3) (width 0.2) (layer "B.Cu") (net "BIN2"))
 (segment (start 104.67 50.87) (end 120.99 50.87) (width 0.2) (layer "F.Cu") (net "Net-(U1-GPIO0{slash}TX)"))
 (segment (start 120.99 50.87) (end 129.62 42.24) (width 0.2) (layer "F.Cu") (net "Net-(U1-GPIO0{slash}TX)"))
 (segment (start 133.124315 36.46) (end 138.83 36.46) (width 0.2) (layer "F.Cu") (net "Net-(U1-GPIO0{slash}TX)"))
 (segment (start 129.62 42.24) (end 129.62 39.964315) (width 0.2) (layer "F.Cu") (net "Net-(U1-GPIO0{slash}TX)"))
 (segment (start 101.94 48.14) (end 104.67 50.87) (width 0.2) (layer "F.Cu") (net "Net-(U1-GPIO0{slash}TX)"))
 (segment (start 138.83 36.46) (end 139.73 37.36) (width 0.2) (layer "F.Cu") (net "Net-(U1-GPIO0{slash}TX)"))
 (segment (start 129.62 39.964315) (end 133.124315 36.46) (width 0.2) (layer "F.Cu") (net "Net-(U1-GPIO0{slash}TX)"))
 (segment (start 120.63 39.113654) (end 120.63 45.615) (width 0.2) (layer "F.Cu") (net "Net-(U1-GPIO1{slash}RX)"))
 (segment (start 131.51 37.15) (end 131.22 37.44) (width 0.2) (layer "F.Cu") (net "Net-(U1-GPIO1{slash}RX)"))
 (segment (start 122.656346 37.8) (end 121.943654 37.8) (width 0.2) (layer "F.Cu") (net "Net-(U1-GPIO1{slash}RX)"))
 (segment (start 120.63 45.615) (end 118.105 48.14) (width 0.2) (layer "F.Cu") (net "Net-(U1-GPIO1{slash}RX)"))
 (segment (start 123.016346 37.44) (end 122.656346 37.8) (width 0.2) (layer "F.Cu") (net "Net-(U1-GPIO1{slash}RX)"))
 (segment (start 121.943654 37.8) (end 120.63 39.113654) (width 0.2) (layer "F.Cu") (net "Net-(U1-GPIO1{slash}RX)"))
 (segment (start 131.22 37.44) (end 123.016346 37.44) (width 0.2) (layer "F.Cu") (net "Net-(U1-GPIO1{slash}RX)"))
 (via (at 131.51 37.15) (size 0.6) (drill 0.3) (layers "F.Cu" "B.Cu") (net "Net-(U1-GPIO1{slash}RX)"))
 (segment (start 131.51 37.75) (end 131.51 37.15) (width 0.2) (layer "B.Cu") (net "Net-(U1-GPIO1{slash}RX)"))
 (segment (start 133.66 39.9) (end 131.51 37.75) (width 0.2) (layer "B.Cu") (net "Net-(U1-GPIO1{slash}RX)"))
 (segment (start 139.73 39.9) (end 133.66 39.9) (width 0.2) (layer "B.Cu") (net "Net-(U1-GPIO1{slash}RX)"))
 (segment (start 131.666346 36.023654) (end 126.54 41.15) (width 0.2) (layer "B.Cu") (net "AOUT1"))
 (segment (start 141.681346 36.023654) (end 131.666346 36.023654) (width 0.2) (layer "B.Cu") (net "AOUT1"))
 (segment (start 143.105 34.6) (end 141.681346 36.023654) (width 0.2) (layer "B.Cu") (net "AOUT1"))
 (segment (start 136.925 45.86) (end 143.105 39.68) (width 0.2) (layer "B.Cu") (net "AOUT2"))
 (segment (start 128.71 45.86) (end 136.925 45.86) (width 0.2) (layer "B.Cu") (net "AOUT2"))
 (segment (start 126.54 43.69) (end 128.71 45.86) (width 0.2) (layer "B.Cu") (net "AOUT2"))
 (segment (start 143.220635 45.86) (end 142.649365 45.86) (width 0.2) (layer "F.Cu") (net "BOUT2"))
 (segment (start 142.005 43.32) (end 143.105 42.22) (width 0.2) (layer "F.Cu") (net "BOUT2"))
 (segment (start 144.270635 47.69) (end 144.270635 46.91) (width 0.2) (layer "F.Cu") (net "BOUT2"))
 (segment (start 144.270635 46.91) (end 143.220635 45.86) (width 0.2) (layer "F.Cu") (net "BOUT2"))
 (segment (start 135.54 48.4) (end 143.560635 48.4) (width 0.2) (layer "F.Cu") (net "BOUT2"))
 (segment (start 130.77 43.63) (end 135.54 48.4) (width 0.2) (layer "F.Cu") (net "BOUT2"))
 (segment (start 142.649365 45.86) (end 142.005 45.215635) (width 0.2) (layer "F.Cu") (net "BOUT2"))
 (segment (start 142.005 45.215635) (end 142.005 43.32) (width 0.2) (layer "F.Cu") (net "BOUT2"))
 (segment (start 143.560635 48.4) (end 144.270635 47.69) (width 0.2) (layer "F.Cu") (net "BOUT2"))
 (segment (start 136.28 36.86) (end 133.29 36.86) (width 0.2) (layer "F.Cu") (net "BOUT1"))
 (segment (start 133.29 36.86) (end 130.77 39.38) (width 0.2) (layer "F.Cu") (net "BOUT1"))
 (segment (start 130.77 39.38) (end 130.77 41.09) (width 0.2) (layer "F.Cu") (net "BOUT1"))
 (segment (start 137.2 41.395) (end 137.2 37.78) (width 0.2) (layer "F.Cu") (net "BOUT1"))
 (segment (start 137.2 37.78) (end 136.28 36.86) (width 0.2) (layer "F.Cu") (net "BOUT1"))
 (segment (start 143.105 47.3) (end 137.2 41.395) (width 0.2) (layer "F.Cu") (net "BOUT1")))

